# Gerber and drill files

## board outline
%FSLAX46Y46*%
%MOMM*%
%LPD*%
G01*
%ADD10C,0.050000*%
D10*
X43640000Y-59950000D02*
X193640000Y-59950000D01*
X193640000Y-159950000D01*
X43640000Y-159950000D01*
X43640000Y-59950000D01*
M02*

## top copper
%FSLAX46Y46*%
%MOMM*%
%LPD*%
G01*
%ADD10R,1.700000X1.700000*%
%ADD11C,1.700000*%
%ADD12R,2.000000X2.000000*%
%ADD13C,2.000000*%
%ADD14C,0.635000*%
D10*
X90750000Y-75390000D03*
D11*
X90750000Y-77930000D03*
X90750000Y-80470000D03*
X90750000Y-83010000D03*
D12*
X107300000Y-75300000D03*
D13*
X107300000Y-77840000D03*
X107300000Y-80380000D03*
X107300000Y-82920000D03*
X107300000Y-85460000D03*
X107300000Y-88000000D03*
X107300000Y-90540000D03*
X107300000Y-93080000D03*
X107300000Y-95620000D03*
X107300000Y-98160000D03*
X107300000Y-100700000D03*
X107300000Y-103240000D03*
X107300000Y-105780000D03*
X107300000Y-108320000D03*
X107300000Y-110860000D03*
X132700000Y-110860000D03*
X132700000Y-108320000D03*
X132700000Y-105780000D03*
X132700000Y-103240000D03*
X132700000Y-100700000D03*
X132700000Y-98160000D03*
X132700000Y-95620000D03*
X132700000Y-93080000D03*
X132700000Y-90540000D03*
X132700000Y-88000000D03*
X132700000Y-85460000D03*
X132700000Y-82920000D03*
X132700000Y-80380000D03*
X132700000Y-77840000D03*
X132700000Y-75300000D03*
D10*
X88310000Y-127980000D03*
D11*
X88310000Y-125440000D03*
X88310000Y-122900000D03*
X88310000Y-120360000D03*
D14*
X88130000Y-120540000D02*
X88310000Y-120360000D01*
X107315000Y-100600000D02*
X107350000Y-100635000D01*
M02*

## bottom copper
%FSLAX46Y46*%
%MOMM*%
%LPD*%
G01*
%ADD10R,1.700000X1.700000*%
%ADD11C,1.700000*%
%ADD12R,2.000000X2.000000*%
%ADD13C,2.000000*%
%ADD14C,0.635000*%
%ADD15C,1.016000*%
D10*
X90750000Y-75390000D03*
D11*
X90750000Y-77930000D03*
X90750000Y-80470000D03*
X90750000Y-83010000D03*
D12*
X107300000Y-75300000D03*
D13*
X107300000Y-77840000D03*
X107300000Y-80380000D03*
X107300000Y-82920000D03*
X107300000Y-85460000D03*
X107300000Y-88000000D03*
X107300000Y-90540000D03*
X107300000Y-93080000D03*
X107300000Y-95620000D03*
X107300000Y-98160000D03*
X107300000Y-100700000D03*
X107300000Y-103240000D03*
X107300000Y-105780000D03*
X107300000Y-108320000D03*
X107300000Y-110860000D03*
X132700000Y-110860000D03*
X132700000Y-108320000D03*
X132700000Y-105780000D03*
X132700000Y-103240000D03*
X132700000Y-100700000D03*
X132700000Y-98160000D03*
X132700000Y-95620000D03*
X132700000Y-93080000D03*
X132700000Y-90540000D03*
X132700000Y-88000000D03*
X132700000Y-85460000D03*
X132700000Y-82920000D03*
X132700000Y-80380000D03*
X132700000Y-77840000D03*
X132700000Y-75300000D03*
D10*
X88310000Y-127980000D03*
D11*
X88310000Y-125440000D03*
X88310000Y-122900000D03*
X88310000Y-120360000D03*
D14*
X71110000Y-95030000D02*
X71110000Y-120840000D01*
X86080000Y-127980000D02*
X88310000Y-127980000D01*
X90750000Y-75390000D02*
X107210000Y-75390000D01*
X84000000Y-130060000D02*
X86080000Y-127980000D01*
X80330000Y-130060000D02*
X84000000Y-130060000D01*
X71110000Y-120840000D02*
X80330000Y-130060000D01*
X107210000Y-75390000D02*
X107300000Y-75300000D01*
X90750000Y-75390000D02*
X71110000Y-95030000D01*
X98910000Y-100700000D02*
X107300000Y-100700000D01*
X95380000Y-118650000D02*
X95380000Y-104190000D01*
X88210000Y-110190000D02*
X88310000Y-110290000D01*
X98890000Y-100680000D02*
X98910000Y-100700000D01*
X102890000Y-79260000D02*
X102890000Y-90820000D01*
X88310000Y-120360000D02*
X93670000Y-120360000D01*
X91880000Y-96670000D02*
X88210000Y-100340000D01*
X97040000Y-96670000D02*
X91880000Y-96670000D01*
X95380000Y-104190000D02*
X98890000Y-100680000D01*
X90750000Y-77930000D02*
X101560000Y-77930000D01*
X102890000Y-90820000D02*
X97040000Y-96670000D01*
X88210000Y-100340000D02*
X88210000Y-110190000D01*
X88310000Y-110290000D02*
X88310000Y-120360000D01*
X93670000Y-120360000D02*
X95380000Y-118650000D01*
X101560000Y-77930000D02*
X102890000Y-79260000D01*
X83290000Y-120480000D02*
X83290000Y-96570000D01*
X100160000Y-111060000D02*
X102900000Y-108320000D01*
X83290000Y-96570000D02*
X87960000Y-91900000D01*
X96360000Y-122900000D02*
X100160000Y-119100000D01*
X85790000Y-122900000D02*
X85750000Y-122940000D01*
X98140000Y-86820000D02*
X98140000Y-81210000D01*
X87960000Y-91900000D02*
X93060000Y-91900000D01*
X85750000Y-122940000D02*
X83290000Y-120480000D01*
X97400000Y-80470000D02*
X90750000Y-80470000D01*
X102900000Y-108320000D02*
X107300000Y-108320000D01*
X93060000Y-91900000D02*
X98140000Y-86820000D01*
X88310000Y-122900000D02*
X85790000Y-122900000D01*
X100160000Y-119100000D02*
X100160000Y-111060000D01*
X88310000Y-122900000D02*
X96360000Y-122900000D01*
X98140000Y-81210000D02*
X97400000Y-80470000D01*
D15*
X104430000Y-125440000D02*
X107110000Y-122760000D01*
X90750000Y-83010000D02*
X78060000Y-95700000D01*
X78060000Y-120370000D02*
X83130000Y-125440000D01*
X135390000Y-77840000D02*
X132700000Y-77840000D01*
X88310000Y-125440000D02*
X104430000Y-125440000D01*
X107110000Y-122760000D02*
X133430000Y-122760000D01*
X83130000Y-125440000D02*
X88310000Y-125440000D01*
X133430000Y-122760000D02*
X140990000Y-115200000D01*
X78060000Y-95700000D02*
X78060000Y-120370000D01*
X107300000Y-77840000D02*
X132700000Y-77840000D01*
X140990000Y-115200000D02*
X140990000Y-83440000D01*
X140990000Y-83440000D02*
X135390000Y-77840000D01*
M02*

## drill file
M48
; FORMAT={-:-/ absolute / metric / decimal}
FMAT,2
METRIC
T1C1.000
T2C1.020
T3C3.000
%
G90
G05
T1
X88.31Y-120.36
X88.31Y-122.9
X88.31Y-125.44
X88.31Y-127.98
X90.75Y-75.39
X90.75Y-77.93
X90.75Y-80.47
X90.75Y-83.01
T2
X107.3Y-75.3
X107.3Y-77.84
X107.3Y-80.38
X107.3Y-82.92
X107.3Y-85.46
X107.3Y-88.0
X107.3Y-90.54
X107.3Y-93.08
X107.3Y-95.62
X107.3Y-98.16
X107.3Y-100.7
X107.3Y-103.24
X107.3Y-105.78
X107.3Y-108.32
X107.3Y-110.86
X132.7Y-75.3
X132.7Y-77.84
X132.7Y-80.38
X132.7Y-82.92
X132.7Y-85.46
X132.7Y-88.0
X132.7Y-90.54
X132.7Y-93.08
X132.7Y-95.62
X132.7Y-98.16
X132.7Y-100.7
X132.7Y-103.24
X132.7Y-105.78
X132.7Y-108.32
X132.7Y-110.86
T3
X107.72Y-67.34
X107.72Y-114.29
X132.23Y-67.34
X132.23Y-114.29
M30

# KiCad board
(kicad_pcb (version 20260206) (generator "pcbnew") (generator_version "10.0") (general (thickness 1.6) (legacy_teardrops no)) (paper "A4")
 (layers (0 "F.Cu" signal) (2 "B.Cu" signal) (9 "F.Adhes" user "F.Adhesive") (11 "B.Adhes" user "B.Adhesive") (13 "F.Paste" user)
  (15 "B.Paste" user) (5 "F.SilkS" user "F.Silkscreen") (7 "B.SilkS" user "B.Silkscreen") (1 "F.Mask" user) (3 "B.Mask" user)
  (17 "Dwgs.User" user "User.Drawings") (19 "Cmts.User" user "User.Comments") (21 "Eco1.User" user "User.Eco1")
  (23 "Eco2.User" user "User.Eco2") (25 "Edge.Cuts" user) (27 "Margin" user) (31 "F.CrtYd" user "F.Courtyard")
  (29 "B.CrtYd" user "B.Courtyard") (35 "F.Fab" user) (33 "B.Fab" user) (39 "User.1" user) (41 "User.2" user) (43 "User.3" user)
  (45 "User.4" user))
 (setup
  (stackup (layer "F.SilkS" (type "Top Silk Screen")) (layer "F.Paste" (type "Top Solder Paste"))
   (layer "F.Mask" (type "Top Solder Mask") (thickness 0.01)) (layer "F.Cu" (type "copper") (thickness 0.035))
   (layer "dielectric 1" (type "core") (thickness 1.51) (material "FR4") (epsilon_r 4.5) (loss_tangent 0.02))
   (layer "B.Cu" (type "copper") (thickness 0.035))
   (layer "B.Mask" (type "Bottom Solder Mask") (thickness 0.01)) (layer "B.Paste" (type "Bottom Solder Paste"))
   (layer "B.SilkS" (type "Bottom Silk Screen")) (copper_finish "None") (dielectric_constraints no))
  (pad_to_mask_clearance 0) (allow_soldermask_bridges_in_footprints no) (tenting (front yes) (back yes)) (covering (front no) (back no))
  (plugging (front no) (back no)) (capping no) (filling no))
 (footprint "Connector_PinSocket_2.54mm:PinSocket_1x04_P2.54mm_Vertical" (layer "F.Cu") (at 90.75 75.39)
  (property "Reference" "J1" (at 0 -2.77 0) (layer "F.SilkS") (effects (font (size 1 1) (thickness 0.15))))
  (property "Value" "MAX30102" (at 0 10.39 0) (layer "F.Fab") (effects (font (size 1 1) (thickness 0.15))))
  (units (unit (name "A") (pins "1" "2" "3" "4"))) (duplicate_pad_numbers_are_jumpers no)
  (pad "1" thru_hole rect (at 0 0) (size 1.7 1.7) (drill 1) (layers "*.Cu" "*.Mask") (remove_unused_layers no) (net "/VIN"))
  (pad "2" thru_hole circle (at 0 2.54) (size 1.7 1.7) (drill 1) (layers "*.Cu" "*.Mask") (remove_unused_layers no) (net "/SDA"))
  (pad "3" thru_hole circle (at 0 5.08) (size 1.7 1.7) (drill 1) (layers "*.Cu" "*.Mask") (remove_unused_layers no) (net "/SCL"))
  (pad "4" thru_hole circle (at 0 7.62) (size 1.7 1.7) (drill 1) (layers "*.Cu" "*.Mask") (remove_unused_layers no) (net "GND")))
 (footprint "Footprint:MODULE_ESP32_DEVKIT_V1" (layer "F.Cu") (at 120 90.815)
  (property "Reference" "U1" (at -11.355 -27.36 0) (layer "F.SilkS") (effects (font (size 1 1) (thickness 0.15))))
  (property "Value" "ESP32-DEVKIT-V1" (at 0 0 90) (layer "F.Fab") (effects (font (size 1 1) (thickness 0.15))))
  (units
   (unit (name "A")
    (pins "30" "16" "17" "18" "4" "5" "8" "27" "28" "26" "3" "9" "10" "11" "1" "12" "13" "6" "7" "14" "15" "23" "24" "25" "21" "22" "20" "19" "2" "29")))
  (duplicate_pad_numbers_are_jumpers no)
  (pad "" np_thru_hole circle (at -12.28 -23.475) (size 3 3) (drill 3) (layers "*.Cu" "*.Mask"))
  (pad "" np_thru_hole circle (at -12.28 23.475) (size 3 3) (drill 3) (layers "*.Cu" "*.Mask"))
  (pad "" np_thru_hole circle (at 12.23 -23.475) (size 3 3) (drill 3) (layers "*.Cu" "*.Mask"))
  (pad "" np_thru_hole circle (at 12.23 23.475) (size 3 3) (drill 3) (layers "*.Cu" "*.Mask"))
  (pad "1" thru_hole rect (at -12.7 -15.515) (size 2 2) (drill 1.02) (layers "*.Cu" "*.Mask") (remove_unused_layers no) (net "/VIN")
   (solder_mask_margin 0.102))
  (pad "2" thru_hole circle (at -12.7 -12.975) (size 2 2) (drill 1.02) (layers "*.Cu" "*.Mask") (remove_unused_layers no) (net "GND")
   (solder_mask_margin 0.102))
  (pad "3" thru_hole circle (at -12.7 -10.435) (size 2 2) (drill 1.02) (layers "*.Cu" "*.Mask") (remove_unused_layers no)
   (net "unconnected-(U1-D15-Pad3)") (solder_mask_margin 0.102))
  (pad "4" thru_hole circle (at -12.7 -7.895) (size 2 2) (drill 1.02) (layers "*.Cu" "*.Mask") (remove_unused_layers no)
   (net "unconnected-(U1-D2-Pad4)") (solder_mask_margin 0.102))
  (pad "5" thru_hole circle (at -12.7 -5.355) (size 2 2) (drill 1.02) (layers "*.Cu" "*.Mask") (remove_unused_layers no)
   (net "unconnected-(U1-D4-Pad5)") (solder_mask_margin 0.102))
  (pad "6" thru_hole circle (at -12.7 -2.815) (size 2 2) (drill 1.02) (layers "*.Cu" "*.Mask") (remove_unused_layers no) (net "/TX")
   (solder_mask_margin 0.102))
  (pad "7" thru_hole circle (at -12.7 -0.275) (size 2 2) (drill 1.02) (layers "*.Cu" "*.Mask") (remove_unused_layers no) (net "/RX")
   (solder_mask_margin 0.102))
  (pad "8" thru_hole circle (at -12.7 2.265) (size 2 2) (drill 1.02) (layers "*.Cu" "*.Mask") (remove_unused_layers no)
   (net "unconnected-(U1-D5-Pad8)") (solder_mask_margin 0.102))
  (pad "9" thru_hole circle (at -12.7 4.805) (size 2 2) (drill 1.02) (layers "*.Cu" "*.Mask") (remove_unused_layers no)
   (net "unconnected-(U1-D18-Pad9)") (solder_mask_margin 0.102))
  (pad "10" thru_hole circle (at -12.7 7.345) (size 2 2) (drill 1.02) (layers "*.Cu" "*.Mask") (remove_unused_layers no)
   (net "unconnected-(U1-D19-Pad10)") (solder_mask_margin 0.102))
  (pad "11" thru_hole circle (at -12.7 9.885) (size 2 2) (drill 1.02) (layers "*.Cu" "*.Mask") (remove_unused_layers no) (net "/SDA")
   (solder_mask_margin 0.102))
  (pad "12" thru_hole circle (at -12.7 12.425) (size 2 2) (drill 1.02) (layers "*.Cu" "*.Mask") (remove_unused_layers no)
   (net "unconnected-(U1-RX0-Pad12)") (solder_mask_margin 0.102))
  (pad "13" thru_hole circle (at -12.7 14.965) (size 2 2) (drill 1.02) (layers "*.Cu" "*.Mask") (remove_unused_layers no)
   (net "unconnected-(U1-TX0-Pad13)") (solder_mask_margin 0.102))
  (pad "14" thru_hole circle (at -12.7 17.505) (size 2 2) (drill 1.02) (layers "*.Cu" "*.Mask") (remove_unused_layers no) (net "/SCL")
   (solder_mask_margin 0.102))
  (pad "15" thru_hole circle (at -12.7 20.045) (size 2 2) (drill 1.02) (layers "*.Cu" "*.Mask") (remove_unused_layers no)
   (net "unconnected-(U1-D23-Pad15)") (solder_mask_margin 0.102))
  (pad "16" thru_hole circle (at 12.7 20.045) (size 2 2) (drill 1.02) (layers "*.Cu" "*.Mask") (remove_unused_layers no)
   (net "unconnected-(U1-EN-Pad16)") (solder_mask_margin 0.102))
  (pad "17" thru_hole circle (at 12.7 17.505) (size 2 2) (drill 1.02) (layers "*.Cu" "*.Mask") (remove_unused_layers no)
   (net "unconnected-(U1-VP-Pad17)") (solder_mask_margin 0.102))
  (pad "18" thru_hole circle (at 12.7 14.965) (size 2 2) (drill 1.02) (layers "*.Cu" "*.Mask") (remove_unused_layers no)
   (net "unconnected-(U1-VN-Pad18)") (solder_mask_margin 0.102))
  (pad "19" thru_hole circle (at 12.7 12.425) (size 2 2) (drill 1.02) (layers "*.Cu" "*.Mask") (remove_unused_layers no)
   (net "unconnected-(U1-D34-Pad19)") (solder_mask_margin 0.102))
  (pad "20" thru_hole circle (at 12.7 9.885) (size 2 2) (drill 1.02) (layers "*.Cu" "*.Mask") (remove_unused_layers no)
   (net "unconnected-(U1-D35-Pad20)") (solder_mask_margin 0.102))
  (pad "21" thru_hole circle (at 12.7 7.345) (size 2 2) (drill 1.02) (layers "*.Cu" "*.Mask") (remove_unused_layers no)
   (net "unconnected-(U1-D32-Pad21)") (solder_mask_margin 0.102))
  (pad "22" thru_hole circle (at 12.7 4.805) (size 2 2) (drill 1.02) (layers "*.Cu" "*.Mask") (remove_unused_layers no)
   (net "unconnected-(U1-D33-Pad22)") (solder_mask_margin 0.102))
  (pad "23" thru_hole circle (at 12.7 2.265) (size 2 2) (drill 1.02) (layers "*.Cu" "*.Mask") (remove_unused_layers no)
   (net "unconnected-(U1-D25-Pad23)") (solder_mask_margin 0.102))
  (pad "24" thru_hole circle (at 12.7 -0.275) (size 2 2) (drill 1.02) (layers "*.Cu" "*.Mask") (remove_unused_layers no)
   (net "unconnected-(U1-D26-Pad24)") (solder_mask_margin 0.102))
  (pad "25" thru_hole circle (at 12.7 -2.815) (size 2 2) (drill 1.02) (layers "*.Cu" "*.Mask") (remove_unused_layers no)
   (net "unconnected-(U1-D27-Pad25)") (solder_mask_margin 0.102))
  (pad "26" thru_hole circle (at 12.7 -5.355) (size 2 2) (drill 1.02) (layers "*.Cu" "*.Mask") (remove_unused_layers no)
   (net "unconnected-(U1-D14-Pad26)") (solder_mask_margin 0.102))
  (pad "27" thru_hole circle (at 12.7 -7.895) (size 2 2) (drill 1.02) (layers "*.Cu" "*.Mask") (remove_unused_layers no)
   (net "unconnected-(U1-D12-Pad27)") (solder_mask_margin 0.102))
  (pad "28" thru_hole circle (at 12.7 -10.435) (size 2 2) (drill 1.02) (layers "*.Cu" "*.Mask") (remove_unused_layers no)
   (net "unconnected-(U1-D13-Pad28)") (solder_mask_margin 0.102))
  (pad "29" thru_hole circle (at 12.7 -12.975) (size 2 2) (drill 1.02) (layers "*.Cu" "*.Mask") (remove_unused_layers no) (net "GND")
   (solder_mask_margin 0.102))
  (pad "30" thru_hole circle (at 12.7 -15.515) (size 2 2) (drill 1.02) (layers "*.Cu" "*.Mask") (remove_unused_layers no) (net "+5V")
   (solder_mask_margin 0.102))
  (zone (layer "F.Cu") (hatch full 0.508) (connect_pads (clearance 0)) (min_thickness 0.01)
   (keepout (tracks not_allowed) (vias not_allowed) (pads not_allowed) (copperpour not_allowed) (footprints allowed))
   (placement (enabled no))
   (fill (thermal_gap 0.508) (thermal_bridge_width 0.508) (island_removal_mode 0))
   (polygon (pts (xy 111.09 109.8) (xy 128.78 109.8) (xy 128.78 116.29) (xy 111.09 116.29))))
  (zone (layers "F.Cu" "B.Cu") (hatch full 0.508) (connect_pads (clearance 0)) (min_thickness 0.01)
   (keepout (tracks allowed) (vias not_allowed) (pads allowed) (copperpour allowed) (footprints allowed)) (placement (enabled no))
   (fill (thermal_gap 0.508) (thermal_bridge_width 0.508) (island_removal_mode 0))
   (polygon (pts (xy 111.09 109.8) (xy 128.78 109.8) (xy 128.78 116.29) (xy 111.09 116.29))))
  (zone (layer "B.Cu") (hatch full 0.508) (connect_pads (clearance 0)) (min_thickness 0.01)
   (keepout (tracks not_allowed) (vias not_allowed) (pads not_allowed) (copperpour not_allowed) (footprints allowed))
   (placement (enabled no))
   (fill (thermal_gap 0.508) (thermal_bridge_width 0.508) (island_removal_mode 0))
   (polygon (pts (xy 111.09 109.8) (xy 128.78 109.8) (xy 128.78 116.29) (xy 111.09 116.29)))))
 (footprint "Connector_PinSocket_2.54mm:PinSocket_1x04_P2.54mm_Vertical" (layer "F.Cu") (at 88.31 127.98 180)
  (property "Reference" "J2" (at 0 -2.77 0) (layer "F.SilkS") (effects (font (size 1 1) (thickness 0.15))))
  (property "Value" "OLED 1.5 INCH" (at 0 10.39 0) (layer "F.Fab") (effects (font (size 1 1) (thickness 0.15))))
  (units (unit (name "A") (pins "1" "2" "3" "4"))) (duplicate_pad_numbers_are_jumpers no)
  (pad "1" thru_hole rect (at 0 0 180) (size 1.7 1.7) (drill 1) (layers "*.Cu" "*.Mask") (remove_unused_layers no) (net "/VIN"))
  (pad "2" thru_hole circle (at 0 2.54 180) (size 1.7 1.7) (drill 1) (layers "*.Cu" "*.Mask") (remove_unused_layers no) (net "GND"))
  (pad "3" thru_hole circle (at 0 5.08 180) (size 1.7 1.7) (drill 1) (layers "*.Cu" "*.Mask") (remove_unused_layers no) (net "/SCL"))
  (pad "4" thru_hole circle (at 0 7.62 180) (size 1.7 1.7) (drill 1) (layers "*.Cu" "*.Mask") (remove_unused_layers no) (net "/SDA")))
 (gr_rect (start 43.64 59.95) (end 193.64 159.95) (stroke (width 0.05) (type solid)) (fill no) (layer "Edge.Cuts"))
 (segment (start 71.11 95.03) (end 71.11 120.84) (width 0.635) (layer "B.Cu") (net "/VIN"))
 (segment (start 86.08 127.98) (end 88.31 127.98) (width 0.635) (layer "B.Cu") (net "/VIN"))
 (segment (start 90.75 75.39) (end 107.21 75.39) (width 0.635) (layer "B.Cu") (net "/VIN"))
 (segment (start 84 130.06) (end 86.08 127.98) (width 0.635) (layer "B.Cu") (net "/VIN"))
 (segment (start 80.33 130.06) (end 84 130.06) (width 0.635) (layer "B.Cu") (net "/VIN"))
 (segment (start 71.11 120.84) (end 80.33 130.06) (width 0.635) (layer "B.Cu") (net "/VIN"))
 (segment (start 107.21 75.39) (end 107.3 75.3) (width 0.635) (layer "B.Cu") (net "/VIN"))
 (segment (start 90.75 75.39) (end 71.11 95.03) (width 0.635) (layer "B.Cu") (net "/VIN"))
 (segment (start 88.13 120.54) (end 88.31 120.36) (width 0.635) (layer "F.Cu") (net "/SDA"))
 (segment (start 107.315 100.6) (end 107.35 100.635) (width 0.635) (layer "F.Cu") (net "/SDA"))
 (segment (start 98.91 100.7) (end 107.3 100.7) (width 0.635) (layer "B.Cu") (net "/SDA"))
 (segment (start 95.38 118.65) (end 95.38 104.19) (width 0.635) (layer "B.Cu") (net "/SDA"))
 (segment (start 88.21 110.19) (end 88.31 110.29) (width 0.635) (layer "B.Cu") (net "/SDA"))
 (segment (start 98.89 100.68) (end 98.91 100.7) (width 0.635) (layer "B.Cu") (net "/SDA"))
 (segment (start 102.89 79.26) (end 102.89 90.82) (width 0.635) (layer "B.Cu") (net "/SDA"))
 (segment (start 88.31 120.36) (end 93.67 120.36) (width 0.635) (layer "B.Cu") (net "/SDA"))
 (segment (start 91.88 96.67) (end 88.21 100.34) (width 0.635) (layer "B.Cu") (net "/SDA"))
 (segment (start 97.04 96.67) (end 91.88 96.67) (width 0.635) (layer "B.Cu") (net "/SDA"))
 (segment (start 95.38 104.19) (end 98.89 100.68) (width 0.635) (layer "B.Cu") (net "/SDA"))
 (segment (start 90.75 77.93) (end 101.56 77.93) (width 0.635) (layer "B.Cu") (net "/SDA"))
 (segment (start 102.89 90.82) (end 97.04 96.67) (width 0.635) (layer "B.Cu") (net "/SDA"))
 (segment (start 88.21 100.34) (end 88.21 110.19) (width 0.635) (layer "B.Cu") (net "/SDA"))
 (segment (start 88.31 110.29) (end 88.31 120.36) (width 0.635) (layer "B.Cu") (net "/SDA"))
 (segment (start 93.67 120.36) (end 95.38 118.65) (width 0.635) (layer "B.Cu") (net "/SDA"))
 (segment (start 101.56 77.93) (end 102.89 79.26) (width 0.635) (layer "B.Cu") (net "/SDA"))
 (segment (start 83.29 120.48) (end 83.29 96.57) (width 0.635) (layer "B.Cu") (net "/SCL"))
 (segment (start 100.16 111.06) (end 102.9 108.32) (width 0.635) (layer "B.Cu") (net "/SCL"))
 (segment (start 83.29 96.57) (end 87.96 91.9) (width 0.635) (layer "B.Cu") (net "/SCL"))
 (segment (start 96.36 122.9) (end 100.16 119.1) (width 0.635) (layer "B.Cu") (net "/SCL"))
 (segment (start 85.79 122.9) (end 85.75 122.94) (width 0.635) (layer "B.Cu") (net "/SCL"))
 (segment (start 98.14 86.82) (end 98.14 81.21) (width 0.635) (layer "B.Cu") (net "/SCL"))
 (segment (start 87.96 91.9) (end 93.06 91.9) (width 0.635) (layer "B.Cu") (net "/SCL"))
 (segment (start 85.75 122.94) (end 83.29 120.48) (width 0.635) (layer "B.Cu") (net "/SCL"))
 (segment (start 97.4 80.47) (end 90.75 80.47) (width 0.635) (layer "B.Cu") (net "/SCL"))
 (segment (start 102.9 108.32) (end 107.3 108.32) (width 0.635) (layer "B.Cu") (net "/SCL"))
 (segment (start 93.06 91.9) (end 98.14 86.82) (width 0.635) (layer "B.Cu") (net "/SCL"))
 (segment (start 88.31 122.9) (end 85.79 122.9) (width 0.635) (layer "B.Cu") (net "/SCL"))
 (segment (start 100.16 119.1) (end 100.16 111.06) (width 0.635) (layer "B.Cu") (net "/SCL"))
 (segment (start 88.31 122.9) (end 96.36 122.9) (width 0.635) (layer "B.Cu") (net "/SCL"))
 (segment (start 98.14 81.21) (end 97.4 80.47) (width 0.635) (layer "B.Cu") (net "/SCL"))
 (segment (start 104.43 125.44) (end 107.11 122.76) (width 1.016) (layer "B.Cu") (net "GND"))
 (segment (start 90.75 83.01) (end 78.06 95.7) (width 1.016) (layer "B.Cu") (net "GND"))
 (segment (start 78.06 120.37) (end 83.13 125.44) (width 1.016) (layer "B.Cu") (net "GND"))
 (segment (start 135.39 77.84) (end 132.7 77.84) (width 1.016) (layer "B.Cu") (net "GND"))
 (segment (start 88.31 125.44) (end 104.43 125.44) (width 1.016) (layer "B.Cu") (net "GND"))
 (segment (start 107.11 122.76) (end 133.43 122.76) (width 1.016) (layer "B.Cu") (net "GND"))
 (segment (start 83.13 125.44) (end 88.31 125.44) (width 1.016) (layer "B.Cu") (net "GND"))
 (segment (start 133.43 122.76) (end 140.99 115.2) (width 1.016) (layer "B.Cu") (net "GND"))
 (segment (start 78.06 95.7) (end 78.06 120.37) (width 1.016) (layer "B.Cu") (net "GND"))
 (segment (start 107.3 77.84) (end 132.7 77.84) (width 1.016) (layer "B.Cu") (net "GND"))
 (segment (start 140.99 115.2) (end 140.99 83.44) (width 1.016) (layer "B.Cu") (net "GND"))
 (segment (start 140.99 83.44) (end 135.39 77.84) (width 1.016) (layer "B.Cu") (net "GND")))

